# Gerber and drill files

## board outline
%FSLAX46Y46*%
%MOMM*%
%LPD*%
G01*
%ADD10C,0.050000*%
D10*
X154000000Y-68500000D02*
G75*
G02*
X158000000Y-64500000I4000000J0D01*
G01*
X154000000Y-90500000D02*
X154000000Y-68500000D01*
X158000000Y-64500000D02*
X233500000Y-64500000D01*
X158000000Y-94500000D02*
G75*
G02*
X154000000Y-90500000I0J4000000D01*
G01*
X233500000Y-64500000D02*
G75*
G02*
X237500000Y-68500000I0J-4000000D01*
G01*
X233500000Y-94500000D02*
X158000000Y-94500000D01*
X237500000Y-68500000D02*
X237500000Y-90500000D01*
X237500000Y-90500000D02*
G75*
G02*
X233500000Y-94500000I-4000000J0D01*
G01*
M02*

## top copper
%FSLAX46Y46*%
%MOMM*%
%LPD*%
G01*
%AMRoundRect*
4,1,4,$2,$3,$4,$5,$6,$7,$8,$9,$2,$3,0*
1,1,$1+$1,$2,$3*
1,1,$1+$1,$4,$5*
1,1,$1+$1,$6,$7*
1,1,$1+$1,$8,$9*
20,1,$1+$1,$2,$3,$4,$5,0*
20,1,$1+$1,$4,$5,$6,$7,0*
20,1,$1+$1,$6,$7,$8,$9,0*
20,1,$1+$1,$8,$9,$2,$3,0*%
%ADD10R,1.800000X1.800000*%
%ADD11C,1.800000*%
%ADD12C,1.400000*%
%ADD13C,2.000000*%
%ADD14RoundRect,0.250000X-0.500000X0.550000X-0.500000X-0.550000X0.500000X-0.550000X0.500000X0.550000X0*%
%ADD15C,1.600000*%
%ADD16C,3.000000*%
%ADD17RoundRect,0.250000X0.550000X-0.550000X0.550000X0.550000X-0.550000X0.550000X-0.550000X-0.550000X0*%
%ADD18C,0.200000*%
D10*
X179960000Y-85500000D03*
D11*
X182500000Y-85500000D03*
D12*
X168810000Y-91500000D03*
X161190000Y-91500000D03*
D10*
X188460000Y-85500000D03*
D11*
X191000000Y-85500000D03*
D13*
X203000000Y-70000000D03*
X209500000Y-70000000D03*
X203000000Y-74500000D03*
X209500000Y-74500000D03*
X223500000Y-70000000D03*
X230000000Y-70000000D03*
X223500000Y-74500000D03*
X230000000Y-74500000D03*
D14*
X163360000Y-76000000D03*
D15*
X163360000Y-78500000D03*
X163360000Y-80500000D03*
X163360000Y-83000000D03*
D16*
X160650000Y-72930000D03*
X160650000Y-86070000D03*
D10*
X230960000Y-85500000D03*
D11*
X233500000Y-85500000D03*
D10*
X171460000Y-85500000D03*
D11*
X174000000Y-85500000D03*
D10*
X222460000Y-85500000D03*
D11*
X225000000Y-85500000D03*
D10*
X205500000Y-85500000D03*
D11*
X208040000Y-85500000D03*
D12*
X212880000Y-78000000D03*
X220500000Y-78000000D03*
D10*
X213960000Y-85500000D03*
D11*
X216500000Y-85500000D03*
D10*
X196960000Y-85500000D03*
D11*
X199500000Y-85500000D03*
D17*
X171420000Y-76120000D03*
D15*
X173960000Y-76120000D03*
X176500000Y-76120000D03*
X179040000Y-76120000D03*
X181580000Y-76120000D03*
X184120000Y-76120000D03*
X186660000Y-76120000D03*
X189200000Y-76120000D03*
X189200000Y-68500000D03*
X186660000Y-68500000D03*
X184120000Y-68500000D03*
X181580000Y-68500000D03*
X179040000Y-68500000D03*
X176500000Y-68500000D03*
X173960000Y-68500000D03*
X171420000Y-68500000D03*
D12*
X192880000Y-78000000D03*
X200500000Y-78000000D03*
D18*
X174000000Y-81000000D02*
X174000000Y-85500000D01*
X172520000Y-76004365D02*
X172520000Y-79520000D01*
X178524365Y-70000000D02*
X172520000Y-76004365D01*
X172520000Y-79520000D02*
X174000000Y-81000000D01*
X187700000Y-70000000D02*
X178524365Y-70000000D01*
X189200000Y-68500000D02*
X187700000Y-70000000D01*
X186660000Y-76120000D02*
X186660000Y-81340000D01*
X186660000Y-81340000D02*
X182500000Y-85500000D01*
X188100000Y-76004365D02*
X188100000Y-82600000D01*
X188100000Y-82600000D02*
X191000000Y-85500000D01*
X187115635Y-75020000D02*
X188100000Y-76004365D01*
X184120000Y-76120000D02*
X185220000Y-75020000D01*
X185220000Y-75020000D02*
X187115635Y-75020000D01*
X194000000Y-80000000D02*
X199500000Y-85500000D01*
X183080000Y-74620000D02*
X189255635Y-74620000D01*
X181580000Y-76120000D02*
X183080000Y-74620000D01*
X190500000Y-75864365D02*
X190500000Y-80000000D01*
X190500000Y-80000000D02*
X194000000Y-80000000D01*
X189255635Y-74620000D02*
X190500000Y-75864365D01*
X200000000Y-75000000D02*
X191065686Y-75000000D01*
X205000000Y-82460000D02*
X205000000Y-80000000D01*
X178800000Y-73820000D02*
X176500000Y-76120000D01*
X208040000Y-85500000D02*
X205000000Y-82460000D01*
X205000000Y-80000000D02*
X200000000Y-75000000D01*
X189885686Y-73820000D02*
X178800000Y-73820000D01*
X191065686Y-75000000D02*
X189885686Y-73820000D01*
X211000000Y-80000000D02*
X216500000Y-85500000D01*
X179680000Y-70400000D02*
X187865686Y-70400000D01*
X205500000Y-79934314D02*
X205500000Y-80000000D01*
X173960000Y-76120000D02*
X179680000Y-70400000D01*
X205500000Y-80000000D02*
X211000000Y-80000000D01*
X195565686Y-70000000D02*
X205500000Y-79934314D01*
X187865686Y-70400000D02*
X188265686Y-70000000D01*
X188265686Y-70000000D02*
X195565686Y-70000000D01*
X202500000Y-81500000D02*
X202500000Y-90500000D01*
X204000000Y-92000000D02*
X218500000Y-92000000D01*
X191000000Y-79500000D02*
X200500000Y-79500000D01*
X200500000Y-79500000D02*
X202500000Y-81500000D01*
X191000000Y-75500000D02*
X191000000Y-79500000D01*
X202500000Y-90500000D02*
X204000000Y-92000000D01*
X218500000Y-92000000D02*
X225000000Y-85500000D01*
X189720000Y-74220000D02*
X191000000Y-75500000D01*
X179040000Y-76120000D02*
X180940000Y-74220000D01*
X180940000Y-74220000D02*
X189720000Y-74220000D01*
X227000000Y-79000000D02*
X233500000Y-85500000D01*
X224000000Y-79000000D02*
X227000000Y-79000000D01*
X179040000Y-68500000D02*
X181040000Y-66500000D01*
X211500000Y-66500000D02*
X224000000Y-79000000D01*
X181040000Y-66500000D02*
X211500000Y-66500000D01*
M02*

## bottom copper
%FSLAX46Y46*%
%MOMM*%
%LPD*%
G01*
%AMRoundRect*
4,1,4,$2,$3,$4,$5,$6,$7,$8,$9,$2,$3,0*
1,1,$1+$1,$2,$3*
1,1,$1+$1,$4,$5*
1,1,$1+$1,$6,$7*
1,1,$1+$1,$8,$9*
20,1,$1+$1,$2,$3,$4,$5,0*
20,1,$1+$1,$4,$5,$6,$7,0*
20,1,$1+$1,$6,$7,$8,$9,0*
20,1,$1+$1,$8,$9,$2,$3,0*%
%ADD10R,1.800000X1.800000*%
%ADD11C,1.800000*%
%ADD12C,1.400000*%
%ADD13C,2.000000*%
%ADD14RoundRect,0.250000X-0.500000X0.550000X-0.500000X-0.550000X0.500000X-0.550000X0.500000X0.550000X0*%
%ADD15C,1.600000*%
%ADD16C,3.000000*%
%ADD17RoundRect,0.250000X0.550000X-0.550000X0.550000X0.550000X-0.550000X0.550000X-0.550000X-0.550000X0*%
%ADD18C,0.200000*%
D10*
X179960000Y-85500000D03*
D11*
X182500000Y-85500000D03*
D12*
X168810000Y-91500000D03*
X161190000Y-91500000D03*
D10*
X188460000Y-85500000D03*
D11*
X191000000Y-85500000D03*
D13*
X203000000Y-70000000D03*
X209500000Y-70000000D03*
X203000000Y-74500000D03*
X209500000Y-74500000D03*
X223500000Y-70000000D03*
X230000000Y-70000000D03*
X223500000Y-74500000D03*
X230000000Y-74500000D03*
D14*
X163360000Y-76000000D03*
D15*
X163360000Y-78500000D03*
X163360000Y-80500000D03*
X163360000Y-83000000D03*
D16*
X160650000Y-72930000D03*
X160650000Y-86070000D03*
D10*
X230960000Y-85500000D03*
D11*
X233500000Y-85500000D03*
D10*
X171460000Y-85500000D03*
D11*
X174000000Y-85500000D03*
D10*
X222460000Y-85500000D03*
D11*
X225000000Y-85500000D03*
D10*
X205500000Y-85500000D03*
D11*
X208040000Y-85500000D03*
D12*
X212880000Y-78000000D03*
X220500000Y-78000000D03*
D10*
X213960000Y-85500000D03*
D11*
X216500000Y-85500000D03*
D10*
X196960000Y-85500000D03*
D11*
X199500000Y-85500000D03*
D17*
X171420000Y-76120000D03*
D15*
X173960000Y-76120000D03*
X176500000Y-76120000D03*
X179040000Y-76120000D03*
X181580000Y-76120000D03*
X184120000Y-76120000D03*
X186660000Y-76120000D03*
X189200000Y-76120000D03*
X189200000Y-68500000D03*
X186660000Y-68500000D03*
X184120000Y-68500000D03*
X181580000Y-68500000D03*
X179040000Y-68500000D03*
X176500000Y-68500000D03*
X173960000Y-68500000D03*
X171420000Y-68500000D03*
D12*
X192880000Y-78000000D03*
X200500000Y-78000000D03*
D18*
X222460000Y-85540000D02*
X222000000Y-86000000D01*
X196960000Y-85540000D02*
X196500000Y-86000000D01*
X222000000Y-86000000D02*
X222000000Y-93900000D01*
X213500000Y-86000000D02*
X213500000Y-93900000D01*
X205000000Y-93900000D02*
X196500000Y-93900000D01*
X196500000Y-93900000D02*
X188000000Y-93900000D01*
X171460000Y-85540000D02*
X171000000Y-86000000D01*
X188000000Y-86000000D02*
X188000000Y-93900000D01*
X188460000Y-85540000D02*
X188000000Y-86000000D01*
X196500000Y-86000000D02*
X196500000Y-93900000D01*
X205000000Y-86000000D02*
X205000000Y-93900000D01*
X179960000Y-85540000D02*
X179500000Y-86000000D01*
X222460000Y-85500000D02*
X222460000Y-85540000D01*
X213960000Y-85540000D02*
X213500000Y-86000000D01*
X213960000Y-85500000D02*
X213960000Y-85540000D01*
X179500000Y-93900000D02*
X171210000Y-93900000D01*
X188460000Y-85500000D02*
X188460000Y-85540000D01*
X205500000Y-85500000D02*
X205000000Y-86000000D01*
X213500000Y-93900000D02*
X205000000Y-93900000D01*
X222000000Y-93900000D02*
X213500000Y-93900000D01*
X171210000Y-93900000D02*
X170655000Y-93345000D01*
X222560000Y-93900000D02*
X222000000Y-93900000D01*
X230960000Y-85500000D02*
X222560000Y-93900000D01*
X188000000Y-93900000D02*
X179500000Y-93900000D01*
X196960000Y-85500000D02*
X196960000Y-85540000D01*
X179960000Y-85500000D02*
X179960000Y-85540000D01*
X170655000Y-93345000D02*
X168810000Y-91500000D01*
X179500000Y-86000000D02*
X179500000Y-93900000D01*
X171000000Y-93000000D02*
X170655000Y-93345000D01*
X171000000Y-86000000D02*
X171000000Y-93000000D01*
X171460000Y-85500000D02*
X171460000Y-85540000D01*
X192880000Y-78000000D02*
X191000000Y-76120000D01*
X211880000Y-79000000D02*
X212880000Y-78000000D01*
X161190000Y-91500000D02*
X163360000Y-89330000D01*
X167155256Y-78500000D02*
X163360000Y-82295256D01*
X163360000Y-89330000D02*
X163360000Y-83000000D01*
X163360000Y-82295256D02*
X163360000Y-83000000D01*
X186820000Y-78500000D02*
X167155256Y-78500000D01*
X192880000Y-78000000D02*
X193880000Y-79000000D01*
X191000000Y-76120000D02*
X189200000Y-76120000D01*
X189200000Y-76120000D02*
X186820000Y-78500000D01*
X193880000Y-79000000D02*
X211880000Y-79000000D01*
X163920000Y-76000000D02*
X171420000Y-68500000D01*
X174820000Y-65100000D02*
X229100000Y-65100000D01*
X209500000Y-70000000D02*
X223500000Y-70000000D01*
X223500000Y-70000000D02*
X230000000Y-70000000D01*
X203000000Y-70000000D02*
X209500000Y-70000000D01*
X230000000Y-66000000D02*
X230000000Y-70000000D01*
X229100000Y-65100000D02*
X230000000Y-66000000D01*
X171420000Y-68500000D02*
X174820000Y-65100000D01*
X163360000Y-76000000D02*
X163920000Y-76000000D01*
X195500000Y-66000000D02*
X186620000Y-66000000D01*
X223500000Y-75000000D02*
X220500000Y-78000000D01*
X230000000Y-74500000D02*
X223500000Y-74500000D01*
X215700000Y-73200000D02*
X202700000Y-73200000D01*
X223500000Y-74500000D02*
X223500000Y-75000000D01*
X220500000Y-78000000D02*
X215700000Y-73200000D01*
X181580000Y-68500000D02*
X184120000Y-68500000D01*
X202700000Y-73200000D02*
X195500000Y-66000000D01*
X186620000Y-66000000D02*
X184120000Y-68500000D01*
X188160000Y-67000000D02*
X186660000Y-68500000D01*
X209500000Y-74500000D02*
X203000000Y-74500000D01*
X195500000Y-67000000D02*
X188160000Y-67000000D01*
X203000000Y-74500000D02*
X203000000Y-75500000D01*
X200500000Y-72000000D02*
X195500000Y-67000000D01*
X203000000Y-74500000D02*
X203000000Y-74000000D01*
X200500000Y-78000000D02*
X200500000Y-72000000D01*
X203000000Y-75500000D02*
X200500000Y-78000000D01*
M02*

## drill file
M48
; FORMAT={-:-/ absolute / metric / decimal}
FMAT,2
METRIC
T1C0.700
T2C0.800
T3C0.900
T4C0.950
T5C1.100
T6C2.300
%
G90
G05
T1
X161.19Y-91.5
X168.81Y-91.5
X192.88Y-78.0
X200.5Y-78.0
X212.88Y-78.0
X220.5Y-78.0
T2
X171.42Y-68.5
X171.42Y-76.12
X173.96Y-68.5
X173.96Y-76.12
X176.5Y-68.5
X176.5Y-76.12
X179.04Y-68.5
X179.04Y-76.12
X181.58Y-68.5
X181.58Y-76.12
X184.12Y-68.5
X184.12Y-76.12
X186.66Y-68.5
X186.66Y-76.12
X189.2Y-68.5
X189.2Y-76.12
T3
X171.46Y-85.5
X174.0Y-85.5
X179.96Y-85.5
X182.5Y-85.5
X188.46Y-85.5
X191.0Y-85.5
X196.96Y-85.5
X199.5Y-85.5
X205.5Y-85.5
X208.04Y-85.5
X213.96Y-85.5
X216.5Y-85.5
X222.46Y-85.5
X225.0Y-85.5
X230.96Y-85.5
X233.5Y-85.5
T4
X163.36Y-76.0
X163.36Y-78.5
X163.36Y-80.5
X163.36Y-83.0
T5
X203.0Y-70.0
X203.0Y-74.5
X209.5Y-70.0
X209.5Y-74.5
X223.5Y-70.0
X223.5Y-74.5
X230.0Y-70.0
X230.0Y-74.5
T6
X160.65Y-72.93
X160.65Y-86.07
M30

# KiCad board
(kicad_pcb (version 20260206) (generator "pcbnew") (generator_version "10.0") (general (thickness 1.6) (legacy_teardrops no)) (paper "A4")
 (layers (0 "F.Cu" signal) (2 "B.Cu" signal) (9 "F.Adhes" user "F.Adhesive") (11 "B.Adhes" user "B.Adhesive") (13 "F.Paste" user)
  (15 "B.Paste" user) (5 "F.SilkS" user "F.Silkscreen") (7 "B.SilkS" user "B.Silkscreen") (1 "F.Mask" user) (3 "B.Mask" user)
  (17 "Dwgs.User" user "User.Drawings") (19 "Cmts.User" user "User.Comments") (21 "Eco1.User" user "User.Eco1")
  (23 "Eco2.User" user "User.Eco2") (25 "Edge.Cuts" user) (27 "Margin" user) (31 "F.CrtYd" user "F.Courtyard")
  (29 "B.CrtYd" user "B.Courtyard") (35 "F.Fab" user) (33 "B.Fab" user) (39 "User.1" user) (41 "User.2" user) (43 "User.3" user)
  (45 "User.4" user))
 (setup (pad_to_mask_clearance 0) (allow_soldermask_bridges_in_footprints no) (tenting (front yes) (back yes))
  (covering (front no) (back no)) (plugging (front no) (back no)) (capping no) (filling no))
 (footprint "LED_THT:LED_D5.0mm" (layer "F.Cu") (at 179.96 85.5)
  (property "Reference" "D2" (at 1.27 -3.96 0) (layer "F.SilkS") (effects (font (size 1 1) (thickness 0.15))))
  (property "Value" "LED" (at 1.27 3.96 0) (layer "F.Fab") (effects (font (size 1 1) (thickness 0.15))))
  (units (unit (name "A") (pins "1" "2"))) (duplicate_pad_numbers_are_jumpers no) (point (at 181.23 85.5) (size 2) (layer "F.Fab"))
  (pad "1" thru_hole rect (at 0 0) (size 1.8 1.8) (drill 0.9) (layers "*.Cu" "*.Mask") (remove_unused_layers no) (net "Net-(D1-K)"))
  (pad "2" thru_hole circle (at 2.54 0) (size 1.8 1.8) (drill 0.9) (layers "*.Cu" "*.Mask") (remove_unused_layers no) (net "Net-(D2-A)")))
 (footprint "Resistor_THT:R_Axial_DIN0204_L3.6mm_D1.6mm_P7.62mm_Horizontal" (layer "F.Cu") (at 168.81 91.5 180)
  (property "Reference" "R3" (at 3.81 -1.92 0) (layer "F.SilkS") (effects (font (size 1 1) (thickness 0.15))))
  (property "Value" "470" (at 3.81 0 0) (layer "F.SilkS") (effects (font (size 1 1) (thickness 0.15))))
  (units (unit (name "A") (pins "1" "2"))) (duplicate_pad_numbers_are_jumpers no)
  (pad "1" thru_hole circle (at 0 0 180) (size 1.4 1.4) (drill 0.7) (layers "*.Cu" "*.Mask") (remove_unused_layers no) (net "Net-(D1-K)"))
  (pad "2" thru_hole circle (at 7.62 0 180) (size 1.4 1.4) (drill 0.7) (layers "*.Cu" "*.Mask") (remove_unused_layers no) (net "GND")))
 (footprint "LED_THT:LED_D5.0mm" (layer "F.Cu") (at 188.46 85.5)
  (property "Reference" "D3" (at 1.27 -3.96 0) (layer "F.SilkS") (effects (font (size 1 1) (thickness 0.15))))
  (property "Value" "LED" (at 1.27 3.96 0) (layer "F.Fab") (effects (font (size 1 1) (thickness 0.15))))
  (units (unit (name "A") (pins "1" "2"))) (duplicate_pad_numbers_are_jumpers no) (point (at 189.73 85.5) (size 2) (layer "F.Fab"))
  (pad "1" thru_hole rect (at 0 0) (size 1.8 1.8) (drill 0.9) (layers "*.Cu" "*.Mask") (remove_unused_layers no) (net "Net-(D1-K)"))
  (pad "2" thru_hole circle (at 2.54 0) (size 1.8 1.8) (drill 0.9) (layers "*.Cu" "*.Mask") (remove_unused_layers no) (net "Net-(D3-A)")))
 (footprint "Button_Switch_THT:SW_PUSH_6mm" (layer "F.Cu") (at 203 70)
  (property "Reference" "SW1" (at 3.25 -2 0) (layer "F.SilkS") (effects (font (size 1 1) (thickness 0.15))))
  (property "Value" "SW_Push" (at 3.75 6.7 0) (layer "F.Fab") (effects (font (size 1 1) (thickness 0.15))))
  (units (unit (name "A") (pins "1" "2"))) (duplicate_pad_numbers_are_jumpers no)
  (pad "1" thru_hole circle (at 0 0 90) (size 2 2) (drill 1.1) (layers "*.Cu" "*.Mask") (remove_unused_layers no) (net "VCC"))
  (pad "1" thru_hole circle (at 6.5 0 90) (size 2 2) (drill 1.1) (layers "*.Cu" "*.Mask") (remove_unused_layers no) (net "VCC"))
  (pad "2" thru_hole circle (at 0 4.5 90) (size 2 2) (drill 1.1) (layers "*.Cu" "*.Mask") (remove_unused_layers no) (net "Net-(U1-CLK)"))
  (pad "2" thru_hole circle (at 6.5 4.5 90) (size 2 2) (drill 1.1) (layers "*.Cu" "*.Mask") (remove_unused_layers no) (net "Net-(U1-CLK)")))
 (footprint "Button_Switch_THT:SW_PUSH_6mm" (layer "F.Cu") (at 223.5 70)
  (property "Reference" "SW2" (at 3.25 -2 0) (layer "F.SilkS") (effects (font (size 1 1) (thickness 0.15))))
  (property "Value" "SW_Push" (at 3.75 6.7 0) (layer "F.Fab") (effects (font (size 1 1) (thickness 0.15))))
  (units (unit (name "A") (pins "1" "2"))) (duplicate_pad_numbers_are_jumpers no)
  (pad "1" thru_hole circle (at 0 0 90) (size 2 2) (drill 1.1) (layers "*.Cu" "*.Mask") (remove_unused_layers no) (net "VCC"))
  (pad "1" thru_hole circle (at 6.5 0 90) (size 2 2) (drill 1.1) (layers "*.Cu" "*.Mask") (remove_unused_layers no) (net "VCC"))
  (pad "2" thru_hole circle (at 0 4.5 90) (size 2 2) (drill 1.1) (layers "*.Cu" "*.Mask") (remove_unused_layers no) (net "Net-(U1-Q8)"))
  (pad "2" thru_hole circle (at 6.5 4.5 90) (size 2 2) (drill 1.1) (layers "*.Cu" "*.Mask") (remove_unused_layers no) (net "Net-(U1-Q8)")))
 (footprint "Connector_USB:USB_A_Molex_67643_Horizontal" (layer "F.Cu") (at 163.36 76 -90)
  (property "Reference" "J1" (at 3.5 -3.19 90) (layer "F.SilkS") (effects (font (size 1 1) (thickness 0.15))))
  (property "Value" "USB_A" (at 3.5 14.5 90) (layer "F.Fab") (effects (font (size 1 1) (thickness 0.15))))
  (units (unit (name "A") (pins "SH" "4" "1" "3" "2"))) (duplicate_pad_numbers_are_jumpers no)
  (pad "1" thru_hole roundrect (at 0 0 270) (size 1.6 1.5) (drill 0.95) (layers "*.Cu" "*.Mask") (remove_unused_layers no)
   (roundrect_rratio 0.1666666667) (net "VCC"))
  (pad "2" thru_hole circle (at 2.5 0 270) (size 1.6 1.6) (drill 0.95) (layers "*.Cu" "*.Mask") (remove_unused_layers no)
   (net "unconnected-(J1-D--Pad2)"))
  (pad "3" thru_hole circle (at 4.5 0 270) (size 1.6 1.6) (drill 0.95) (layers "*.Cu" "*.Mask") (remove_unused_layers no)
   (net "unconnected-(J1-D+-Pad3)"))
  (pad "4" thru_hole circle (at 7 0 270) (size 1.6 1.6) (drill 0.95) (layers "*.Cu" "*.Mask") (remove_unused_layers no) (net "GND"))
  (pad "SH" thru_hole circle (at -3.07 2.71 270) (size 3 3) (drill 2.3) (layers "*.Cu" "*.Mask") (remove_unused_layers no)
   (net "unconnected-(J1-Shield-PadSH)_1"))
  (pad "SH" thru_hole circle (at 10.07 2.71 270) (size 3 3) (drill 2.3) (layers "*.Cu" "*.Mask") (remove_unused_layers no)
   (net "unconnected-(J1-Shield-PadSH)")))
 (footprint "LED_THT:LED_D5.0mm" (layer "F.Cu") (at 230.96 85.5)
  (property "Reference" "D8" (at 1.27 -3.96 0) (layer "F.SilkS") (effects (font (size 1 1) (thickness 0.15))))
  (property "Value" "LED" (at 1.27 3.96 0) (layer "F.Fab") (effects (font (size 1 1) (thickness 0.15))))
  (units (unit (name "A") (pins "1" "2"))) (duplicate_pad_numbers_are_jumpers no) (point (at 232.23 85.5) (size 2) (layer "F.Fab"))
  (pad "1" thru_hole rect (at 0 0) (size 1.8 1.8) (drill 0.9) (layers "*.Cu" "*.Mask") (remove_unused_layers no) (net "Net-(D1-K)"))
  (pad "2" thru_hole circle (at 2.54 0) (size 1.8 1.8) (drill 0.9) (layers "*.Cu" "*.Mask") (remove_unused_layers no) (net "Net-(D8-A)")))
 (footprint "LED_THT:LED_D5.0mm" (layer "F.Cu") (at 171.46 85.5)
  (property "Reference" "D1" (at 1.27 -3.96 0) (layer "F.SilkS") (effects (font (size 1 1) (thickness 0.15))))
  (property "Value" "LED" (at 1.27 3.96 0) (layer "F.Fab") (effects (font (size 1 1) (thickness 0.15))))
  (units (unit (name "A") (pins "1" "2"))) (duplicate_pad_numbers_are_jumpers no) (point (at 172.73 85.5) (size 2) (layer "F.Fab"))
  (pad "1" thru_hole rect (at 0 0) (size 1.8 1.8) (drill 0.9) (layers "*.Cu" "*.Mask") (remove_unused_layers no) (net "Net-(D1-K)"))
  (pad "2" thru_hole circle (at 2.54 0) (size 1.8 1.8) (drill 0.9) (layers "*.Cu" "*.Mask") (remove_unused_layers no) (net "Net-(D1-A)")))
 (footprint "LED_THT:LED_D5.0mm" (layer "F.Cu") (at 222.46 85.5)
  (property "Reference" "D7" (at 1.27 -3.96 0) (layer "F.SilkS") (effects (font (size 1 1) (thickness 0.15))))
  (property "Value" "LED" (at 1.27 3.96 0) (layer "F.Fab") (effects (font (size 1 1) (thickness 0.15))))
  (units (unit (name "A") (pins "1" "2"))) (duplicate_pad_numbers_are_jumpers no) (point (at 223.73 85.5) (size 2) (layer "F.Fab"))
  (pad "1" thru_hole rect (at 0 0) (size 1.8 1.8) (drill 0.9) (layers "*.Cu" "*.Mask") (remove_unused_layers no) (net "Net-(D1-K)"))
  (pad "2" thru_hole circle (at 2.54 0) (size 1.8 1.8) (drill 0.9) (layers "*.Cu" "*.Mask") (remove_unused_layers no) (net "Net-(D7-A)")))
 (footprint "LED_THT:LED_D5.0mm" (layer "F.Cu") (at 205.5 85.5)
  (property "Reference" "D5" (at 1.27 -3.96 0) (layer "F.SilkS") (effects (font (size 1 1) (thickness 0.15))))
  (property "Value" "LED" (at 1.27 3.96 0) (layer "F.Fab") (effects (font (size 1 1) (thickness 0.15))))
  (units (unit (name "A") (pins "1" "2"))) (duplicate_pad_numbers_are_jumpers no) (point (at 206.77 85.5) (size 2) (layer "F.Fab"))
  (pad "1" thru_hole rect (at 0 0) (size 1.8 1.8) (drill 0.9) (layers "*.Cu" "*.Mask") (remove_unused_layers no) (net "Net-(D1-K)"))
  (pad "2" thru_hole circle (at 2.54 0) (size 1.8 1.8) (drill 0.9) (layers "*.Cu" "*.Mask") (remove_unused_layers no) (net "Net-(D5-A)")))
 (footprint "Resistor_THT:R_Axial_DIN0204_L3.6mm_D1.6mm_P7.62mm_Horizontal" (layer "F.Cu") (at 212.88 78)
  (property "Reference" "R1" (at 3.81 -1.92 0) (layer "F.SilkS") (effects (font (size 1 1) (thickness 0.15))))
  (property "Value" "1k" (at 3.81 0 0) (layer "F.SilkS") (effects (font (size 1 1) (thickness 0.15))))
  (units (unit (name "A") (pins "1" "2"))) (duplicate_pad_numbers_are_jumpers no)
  (pad "1" thru_hole circle (at 0 0) (size 1.4 1.4) (drill 0.7) (layers "*.Cu" "*.Mask") (remove_unused_layers no) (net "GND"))
  (pad "2" thru_hole circle (at 7.62 0) (size 1.4 1.4) (drill 0.7) (layers "*.Cu" "*.Mask") (remove_unused_layers no) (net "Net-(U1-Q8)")))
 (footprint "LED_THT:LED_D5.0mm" (layer "F.Cu") (at 213.96 85.5)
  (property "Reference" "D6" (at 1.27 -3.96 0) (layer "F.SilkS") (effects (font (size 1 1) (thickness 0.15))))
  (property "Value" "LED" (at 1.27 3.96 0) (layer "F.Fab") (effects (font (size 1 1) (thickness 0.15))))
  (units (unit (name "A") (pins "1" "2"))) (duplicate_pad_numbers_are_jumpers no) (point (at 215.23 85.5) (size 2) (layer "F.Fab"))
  (pad "1" thru_hole rect (at 0 0) (size 1.8 1.8) (drill 0.9) (layers "*.Cu" "*.Mask") (remove_unused_layers no) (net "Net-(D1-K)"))
  (pad "2" thru_hole circle (at 2.54 0) (size 1.8 1.8) (drill 0.9) (layers "*.Cu" "*.Mask") (remove_unused_layers no) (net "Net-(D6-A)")))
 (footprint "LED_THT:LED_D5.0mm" (layer "F.Cu") (at 196.96 85.5)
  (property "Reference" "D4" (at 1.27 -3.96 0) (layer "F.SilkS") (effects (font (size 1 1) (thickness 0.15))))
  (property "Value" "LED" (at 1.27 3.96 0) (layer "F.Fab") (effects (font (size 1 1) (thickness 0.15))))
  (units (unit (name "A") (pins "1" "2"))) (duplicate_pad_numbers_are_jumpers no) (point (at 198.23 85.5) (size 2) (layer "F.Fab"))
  (pad "1" thru_hole rect (at 0 0) (size 1.8 1.8) (drill 0.9) (layers "*.Cu" "*.Mask") (remove_unused_layers no) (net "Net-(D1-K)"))
  (pad "2" thru_hole circle (at 2.54 0) (size 1.8 1.8) (drill 0.9) (layers "*.Cu" "*.Mask") (remove_unused_layers no) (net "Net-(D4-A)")))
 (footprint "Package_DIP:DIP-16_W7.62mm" (layer "F.Cu") (at 171.42 76.12 90)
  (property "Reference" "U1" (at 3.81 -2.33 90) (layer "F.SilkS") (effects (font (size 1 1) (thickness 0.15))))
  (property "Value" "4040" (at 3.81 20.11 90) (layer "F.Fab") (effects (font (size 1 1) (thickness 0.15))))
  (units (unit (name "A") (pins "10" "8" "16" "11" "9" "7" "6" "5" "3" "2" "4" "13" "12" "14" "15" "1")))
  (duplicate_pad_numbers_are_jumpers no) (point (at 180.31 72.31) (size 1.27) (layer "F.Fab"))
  (pad "1" thru_hole roundrect (at 0 0 90) (size 1.6 1.6) (drill 0.8) (layers "*.Cu" "*.Mask") (remove_unused_layers no)
   (roundrect_rratio 0.15625) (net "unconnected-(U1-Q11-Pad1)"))
  (pad "2" thru_hole circle (at 0 2.54 90) (size 1.6 1.6) (drill 0.8) (layers "*.Cu" "*.Mask") (remove_unused_layers no) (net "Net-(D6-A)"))
  (pad "3" thru_hole circle (at 0 5.08 90) (size 1.6 1.6) (drill 0.8) (layers "*.Cu" "*.Mask") (remove_unused_layers no) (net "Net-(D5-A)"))
  (pad "4" thru_hole circle (at 0 7.62 90) (size 1.6 1.6) (drill 0.8) (layers "*.Cu" "*.Mask") (remove_unused_layers no) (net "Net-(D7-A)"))
  (pad "5" thru_hole circle (at 0 10.16 90) (size 1.6 1.6) (drill 0.8) (layers "*.Cu" "*.Mask") (remove_unused_layers no) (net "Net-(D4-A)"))
  (pad "6" thru_hole circle (at 0 12.7 90) (size 1.6 1.6) (drill 0.8) (layers "*.Cu" "*.Mask") (remove_unused_layers no) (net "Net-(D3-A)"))
  (pad "7" thru_hole circle (at 0 15.24 90) (size 1.6 1.6) (drill 0.8) (layers "*.Cu" "*.Mask") (remove_unused_layers no) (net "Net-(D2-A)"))
  (pad "8" thru_hole circle (at 0 17.78 90) (size 1.6 1.6) (drill 0.8) (layers "*.Cu" "*.Mask") (remove_unused_layers no) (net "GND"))
  (pad "9" thru_hole circle (at 7.62 17.78 90) (size 1.6 1.6) (drill 0.8) (layers "*.Cu" "*.Mask") (remove_unused_layers no)
   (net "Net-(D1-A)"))
  (pad "10" thru_hole circle (at 7.62 15.24 90) (size 1.6 1.6) (drill 0.8) (layers "*.Cu" "*.Mask") (remove_unused_layers no)
   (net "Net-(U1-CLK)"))
  (pad "11" thru_hole circle (at 7.62 12.7 90) (size 1.6 1.6) (drill 0.8) (layers "*.Cu" "*.Mask") (remove_unused_layers no)
   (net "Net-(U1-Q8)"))
  (pad "12" thru_hole circle (at 7.62 10.16 90) (size 1.6 1.6) (drill 0.8) (layers "*.Cu" "*.Mask") (remove_unused_layers no)
   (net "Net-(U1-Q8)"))
  (pad "13" thru_hole circle (at 7.62 7.62 90) (size 1.6 1.6) (drill 0.8) (layers "*.Cu" "*.Mask") (remove_unused_layers no)
   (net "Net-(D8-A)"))
  (pad "14" thru_hole circle (at 7.62 5.08 90) (size 1.6 1.6) (drill 0.8) (layers "*.Cu" "*.Mask") (remove_unused_layers no)
   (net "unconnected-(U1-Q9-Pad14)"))
  (pad "15" thru_hole circle (at 7.62 2.54 90) (size 1.6 1.6) (drill 0.8) (layers "*.Cu" "*.Mask") (remove_unused_layers no)
   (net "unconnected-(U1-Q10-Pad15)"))
  (pad "16" thru_hole circle (at 7.62 0 90) (size 1.6 1.6) (drill 0.8) (layers "*.Cu" "*.Mask") (remove_unused_layers no) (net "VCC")))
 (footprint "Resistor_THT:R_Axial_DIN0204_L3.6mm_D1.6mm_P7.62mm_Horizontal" (layer "F.Cu") (at 192.88 78)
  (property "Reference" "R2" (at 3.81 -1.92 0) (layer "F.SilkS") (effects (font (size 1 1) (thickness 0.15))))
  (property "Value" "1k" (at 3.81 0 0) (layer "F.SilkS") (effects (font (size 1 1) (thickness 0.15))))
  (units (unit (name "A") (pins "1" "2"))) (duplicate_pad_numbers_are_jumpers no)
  (pad "1" thru_hole circle (at 0 0) (size 1.4 1.4) (drill 0.7) (layers "*.Cu" "*.Mask") (remove_unused_layers no) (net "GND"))
  (pad "2" thru_hole circle (at 7.62 0) (size 1.4 1.4) (drill 0.7) (layers "*.Cu" "*.Mask") (remove_unused_layers no) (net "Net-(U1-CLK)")))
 (gr_arc (start 154 68.5) (mid 155.171573 65.671573) (end 158 64.5) (stroke (width 0.05) (type default)) (layer "Edge.Cuts"))
 (gr_line (start 154 90.5) (end 154 68.5) (stroke (width 0.05) (type default)) (layer "Edge.Cuts"))
 (gr_line (start 158 64.5) (end 233.5 64.5) (stroke (width 0.05) (type default)) (layer "Edge.Cuts"))
 (gr_arc (start 158 94.5) (mid 155.171573 93.328427) (end 154 90.5) (stroke (width 0.05) (type default)) (layer "Edge.Cuts"))
 (gr_arc (start 233.5 64.5) (mid 236.328427 65.671573) (end 237.5 68.5) (stroke (width 0.05) (type default)) (layer "Edge.Cuts"))
 (gr_line (start 233.5 94.5) (end 158 94.5) (stroke (width 0.05) (type default)) (layer "Edge.Cuts"))
 (gr_line (start 237.5 68.5) (end 237.5 90.5) (stroke (width 0.05) (type default)) (layer "Edge.Cuts"))
 (gr_arc (start 237.5 90.5) (mid 236.328427 93.328427) (end 233.5 94.5) (stroke (width 0.05) (type default)) (layer "Edge.Cuts"))
 (segment (start 222.46 85.54) (end 222 86) (width 0.2) (layer "B.Cu") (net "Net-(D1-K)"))
 (segment (start 196.96 85.54) (end 196.5 86) (width 0.2) (layer "B.Cu") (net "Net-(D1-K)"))
 (segment (start 222 86) (end 222 93.9) (width 0.2) (layer "B.Cu") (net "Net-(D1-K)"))
 (segment (start 213.5 86) (end 213.5 93.9) (width 0.2) (layer "B.Cu") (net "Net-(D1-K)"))
 (segment (start 205 93.9) (end 196.5 93.9) (width 0.2) (layer "B.Cu") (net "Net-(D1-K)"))
 (segment (start 196.5 93.9) (end 188 93.9) (width 0.2) (layer "B.Cu") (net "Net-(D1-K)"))
 (segment (start 171.46 85.54) (end 171 86) (width 0.2) (layer "B.Cu") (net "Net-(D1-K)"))
 (segment (start 188 86) (end 188 93.9) (width 0.2) (layer "B.Cu") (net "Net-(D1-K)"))
 (segment (start 188.46 85.54) (end 188 86) (width 0.2) (layer "B.Cu") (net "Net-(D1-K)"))
 (segment (start 196.5 86) (end 196.5 93.9) (width 0.2) (layer "B.Cu") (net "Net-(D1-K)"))
 (segment (start 205 86) (end 205 93.9) (width 0.2) (layer "B.Cu") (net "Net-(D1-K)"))
 (segment (start 179.96 85.54) (end 179.5 86) (width 0.2) (layer "B.Cu") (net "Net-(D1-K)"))
 (segment (start 222.46 85.5) (end 222.46 85.54) (width 0.2) (layer "B.Cu") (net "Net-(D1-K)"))
 (segment (start 213.96 85.54) (end 213.5 86) (width 0.2) (layer "B.Cu") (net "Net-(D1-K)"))
 (segment (start 213.96 85.5) (end 213.96 85.54) (width 0.2) (layer "B.Cu") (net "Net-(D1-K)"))
 (segment (start 179.5 93.9) (end 171.21 93.9) (width 0.2) (layer "B.Cu") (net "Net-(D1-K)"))
 (segment (start 188.46 85.5) (end 188.46 85.54) (width 0.2) (layer "B.Cu") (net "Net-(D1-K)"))
 (segment (start 205.5 85.5) (end 205 86) (width 0.2) (layer "B.Cu") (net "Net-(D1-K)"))
 (segment (start 213.5 93.9) (end 205 93.9) (width 0.2) (layer "B.Cu") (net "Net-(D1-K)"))
 (segment (start 222 93.9) (end 213.5 93.9) (width 0.2) (layer "B.Cu") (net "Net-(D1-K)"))
 (segment (start 171.21 93.9) (end 170.655 93.345) (width 0.2) (layer "B.Cu") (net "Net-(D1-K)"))
 (segment (start 222.56 93.9) (end 222 93.9) (width 0.2) (layer "B.Cu") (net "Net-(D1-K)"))
 (segment (start 230.96 85.5) (end 222.56 93.9) (width 0.2) (layer "B.Cu") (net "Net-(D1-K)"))
 (segment (start 188 93.9) (end 179.5 93.9) (width 0.2) (layer "B.Cu") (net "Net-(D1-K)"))
 (segment (start 196.96 85.5) (end 196.96 85.54) (width 0.2) (layer "B.Cu") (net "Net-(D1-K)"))
 (segment (start 179.96 85.5) (end 179.96 85.54) (width 0.2) (layer "B.Cu") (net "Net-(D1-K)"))
 (segment (start 170.655 93.345) (end 168.81 91.5) (width 0.2) (layer "B.Cu") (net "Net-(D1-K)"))
 (segment (start 179.5 86) (end 179.5 93.9) (width 0.2) (layer "B.Cu") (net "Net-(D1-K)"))
 (segment (start 171 93) (end 170.655 93.345) (width 0.2) (layer "B.Cu") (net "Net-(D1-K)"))
 (segment (start 171 86) (end 171 93) (width 0.2) (layer "B.Cu") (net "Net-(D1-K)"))
 (segment (start 171.46 85.5) (end 171.46 85.54) (width 0.2) (layer "B.Cu") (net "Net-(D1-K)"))
 (segment (start 174 81) (end 174 85.5) (width 0.2) (layer "F.Cu") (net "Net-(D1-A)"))
 (segment (start 172.52 76.004365) (end 172.52 79.52) (width 0.2) (layer "F.Cu") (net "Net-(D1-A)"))
 (segment (start 178.524365 70) (end 172.52 76.004365) (width 0.2) (layer "F.Cu") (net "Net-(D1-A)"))
 (segment (start 172.52 79.52) (end 174 81) (width 0.2) (layer "F.Cu") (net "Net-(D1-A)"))
 (segment (start 187.7 70) (end 178.524365 70) (width 0.2) (layer "F.Cu") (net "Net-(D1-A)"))
 (segment (start 189.2 68.5) (end 187.7 70) (width 0.2) (layer "F.Cu") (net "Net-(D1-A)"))
 (segment (start 186.66 76.12) (end 186.66 81.34) (width 0.2) (layer "F.Cu") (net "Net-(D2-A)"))
 (segment (start 186.66 81.34) (end 182.5 85.5) (width 0.2) (layer "F.Cu") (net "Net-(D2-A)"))
 (segment (start 188.1 76.004365) (end 188.1 82.6) (width 0.2) (layer "F.Cu") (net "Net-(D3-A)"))
 (segment (start 188.1 82.6) (end 191 85.5) (width 0.2) (layer "F.Cu") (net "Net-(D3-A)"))
 (segment (start 187.115635 75.02) (end 188.1 76.004365) (width 0.2) (layer "F.Cu") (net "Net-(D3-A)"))
 (segment (start 184.12 76.12) (end 185.22 75.02) (width 0.2) (layer "F.Cu") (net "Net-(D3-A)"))
 (segment (start 185.22 75.02) (end 187.115635 75.02) (width 0.2) (layer "F.Cu") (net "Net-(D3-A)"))
 (segment (start 194 80) (end 199.5 85.5) (width 0.2) (layer "F.Cu") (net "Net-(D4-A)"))
 (segment (start 183.08 74.62) (end 189.255635 74.62) (width 0.2) (layer "F.Cu") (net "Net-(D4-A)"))
 (segment (start 181.58 76.12) (end 183.08 74.62) (width 0.2) (layer "F.Cu") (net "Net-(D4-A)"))
 (segment (start 190.5 75.864365) (end 190.5 80) (width 0.2) (layer "F.Cu") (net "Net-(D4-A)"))
 (segment (start 190.5 80) (end 194 80) (width 0.2) (layer "F.Cu") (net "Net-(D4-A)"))
 (segment (start 189.255635 74.62) (end 190.5 75.864365) (width 0.2) (layer "F.Cu") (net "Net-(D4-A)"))
 (segment (start 200 75) (end 191.065686 75) (width 0.2) (layer "F.Cu") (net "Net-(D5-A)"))
 (segment (start 205 82.46) (end 205 80) (width 0.2) (layer "F.Cu") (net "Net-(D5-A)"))
 (segment (start 178.8 73.82) (end 176.5 76.12) (width 0.2) (layer "F.Cu") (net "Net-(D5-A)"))
 (segment (start 208.04 85.5) (end 205 82.46) (width 0.2) (layer "F.Cu") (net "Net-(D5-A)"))
 (segment (start 205 80) (end 200 75) (width 0.2) (layer "F.Cu") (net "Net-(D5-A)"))
 (segment (start 189.885686 73.82) (end 178.8 73.82) (width 0.2) (layer "F.Cu") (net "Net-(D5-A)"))
 (segment (start 191.065686 75) (end 189.885686 73.82) (width 0.2) (layer "F.Cu") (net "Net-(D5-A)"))
 (segment (start 211 80) (end 216.5 85.5) (width 0.2) (layer "F.Cu") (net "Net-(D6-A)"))
 (segment (start 179.68 70.4) (end 187.865686 70.4) (width 0.2) (layer "F.Cu") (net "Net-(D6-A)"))
 (segment (start 205.5 79.934314) (end 205.5 80) (width 0.2) (layer "F.Cu") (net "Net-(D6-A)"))
 (segment (start 173.96 76.12) (end 179.68 70.4) (width 0.2) (layer "F.Cu") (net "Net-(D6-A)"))
 (segment (start 205.5 80) (end 211 80) (width 0.2) (layer "F.Cu") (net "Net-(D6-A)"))
 (segment (start 195.565686 70) (end 205.5 79.934314) (width 0.2) (layer "F.Cu") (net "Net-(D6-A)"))
 (segment (start 187.865686 70.4) (end 188.265686 70) (width 0.2) (layer "F.Cu") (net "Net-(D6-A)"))
 (segment (start 188.265686 70) (end 195.565686 70) (width 0.2) (layer "F.Cu") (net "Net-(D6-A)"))
 (segment (start 202.5 81.5) (end 202.5 90.5) (width 0.2) (layer "F.Cu") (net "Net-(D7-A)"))
 (segment (start 204 92) (end 218.5 92) (width 0.2) (layer "F.Cu") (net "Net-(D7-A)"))
 (segment (start 191 79.5) (end 200.5 79.5) (width 0.2) (layer "F.Cu") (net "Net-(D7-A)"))
 (segment (start 200.5 79.5) (end 202.5 81.5) (width 0.2) (layer "F.Cu") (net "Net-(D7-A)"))
 (segment (start 191 75.5) (end 191 79.5) (width 0.2) (layer "F.Cu") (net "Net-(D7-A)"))
 (segment (start 202.5 90.5) (end 204 92) (width 0.2) (layer "F.Cu") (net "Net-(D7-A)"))
 (segment (start 218.5 92) (end 225 85.5) (width 0.2) (layer "F.Cu") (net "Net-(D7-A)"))
 (segment (start 189.72 74.22) (end 191 75.5) (width 0.2) (layer "F.Cu") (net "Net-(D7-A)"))
 (segment (start 179.04 76.12) (end 180.94 74.22) (width 0.2) (layer "F.Cu") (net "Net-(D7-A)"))
 (segment (start 180.94 74.22) (end 189.72 74.22) (width 0.2) (layer "F.Cu") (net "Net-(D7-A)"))
 (segment (start 227 79) (end 233.5 85.5) (width 0.2) (layer "F.Cu") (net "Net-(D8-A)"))
 (segment (start 224 79) (end 227 79) (width 0.2) (layer "F.Cu") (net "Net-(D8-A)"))
 (segment (start 179.04 68.5) (end 181.04 66.5) (width 0.2) (layer "F.Cu") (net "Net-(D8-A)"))
 (segment (start 211.5 66.5) (end 224 79) (width 0.2) (layer "F.Cu") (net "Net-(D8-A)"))
 (segment (start 181.04 66.5) (end 211.5 66.5) (width 0.2) (layer "F.Cu") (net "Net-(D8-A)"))
 (segment (start 192.88 78) (end 191 76.12) (width 0.2) (layer "B.Cu") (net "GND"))
 (segment (start 211.88 79) (end 212.88 78) (width 0.2) (layer "B.Cu") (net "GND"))
 (segment (start 161.19 91.5) (end 163.36 89.33) (width 0.2) (layer "B.Cu") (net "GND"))
 (segment (start 167.155256 78.5) (end 163.36 82.295256) (width 0.2) (layer "B.Cu") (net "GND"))
 (segment (start 163.36 89.33) (end 163.36 83) (width 0.2) (layer "B.Cu") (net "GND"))
 (segment (start 163.36 82.295256) (end 163.36 83) (width 0.2) (layer "B.Cu") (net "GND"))
 (segment (start 186.82 78.5) (end 167.155256 78.5) (width 0.2) (layer "B.Cu") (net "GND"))
 (segment (start 192.88 78) (end 193.88 79) (width 0.2) (layer "B.Cu") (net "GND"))
 (segment (start 191 76.12) (end 189.2 76.12) (width 0.2) (layer "B.Cu") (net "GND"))
 (segment (start 189.2 76.12) (end 186.82 78.5) (width 0.2) (layer "B.Cu") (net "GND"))
 (segment (start 193.88 79) (end 211.88 79) (width 0.2) (layer "B.Cu") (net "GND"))
 (segment (start 163.92 76) (end 171.42 68.5) (width 0.2) (layer "B.Cu") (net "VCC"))
 (segment (start 174.82 65.1) (end 229.1 65.1) (width 0.2) (layer "B.Cu") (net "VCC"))
 (segment (start 209.5 70) (end 223.5 70) (width 0.2) (layer "B.Cu") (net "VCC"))
 (segment (start 223.5 70) (end 230 70) (width 0.2) (layer "B.Cu") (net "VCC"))
 (segment (start 203 70) (end 209.5 70) (width 0.2) (layer "B.Cu") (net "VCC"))
 (segment (start 230 66) (end 230 70) (width 0.2) (layer "B.Cu") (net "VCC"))
 (segment (start 229.1 65.1) (end 230 66) (width 0.2) (layer "B.Cu") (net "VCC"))
 (segment (start 171.42 68.5) (end 174.82 65.1) (width 0.2) (layer "B.Cu") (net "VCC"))
 (segment (start 163.36 76) (end 163.92 76) (width 0.2) (layer "B.Cu") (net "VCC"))
 (segment (start 195.5 66) (end 186.62 66) (width 0.2) (layer "B.Cu") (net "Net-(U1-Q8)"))
 (segment (start 223.5 75) (end 220.5 78) (width 0.2) (layer "B.Cu") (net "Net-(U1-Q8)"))
 (segment (start 230 74.5) (end 223.5 74.5) (width 0.2) (layer "B.Cu") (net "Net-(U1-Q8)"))
 (segment (start 215.7 73.2) (end 202.7 73.2) (width 0.2) (layer "B.Cu") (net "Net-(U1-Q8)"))
 (segment (start 223.5 74.5) (end 223.5 75) (width 0.2) (layer "B.Cu") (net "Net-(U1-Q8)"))
 (segment (start 220.5 78) (end 215.7 73.2) (width 0.2) (layer "B.Cu") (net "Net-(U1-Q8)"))
 (segment (start 181.58 68.5) (end 184.12 68.5) (width 0.2) (layer "B.Cu") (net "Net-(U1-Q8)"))
 (segment (start 202.7 73.2) (end 195.5 66) (width 0.2) (layer "B.Cu") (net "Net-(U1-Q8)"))
 (segment (start 186.62 66) (end 184.12 68.5) (width 0.2) (layer "B.Cu") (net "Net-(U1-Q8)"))
 (segment (start 188.16 67) (end 186.66 68.5) (width 0.2) (layer "B.Cu") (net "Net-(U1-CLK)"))
 (segment (start 209.5 74.5) (end 203 74.5) (width 0.2) (layer "B.Cu") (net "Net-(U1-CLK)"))
 (segment (start 195.5 67) (end 188.16 67) (width 0.2) (layer "B.Cu") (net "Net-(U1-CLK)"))
 (segment (start 203 74.5) (end 203 75.5) (width 0.2) (layer "B.Cu") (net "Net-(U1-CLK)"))
 (segment (start 200.5 72) (end 195.5 67) (width 0.2) (layer "B.Cu") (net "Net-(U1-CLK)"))
 (segment (start 203 74.5) (end 203 74) (width 0.2) (layer "B.Cu") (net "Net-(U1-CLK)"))
 (segment (start 200.5 78) (end 200.5 72) (width 0.2) (layer "B.Cu") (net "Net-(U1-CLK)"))
 (segment (start 203 75.5) (end 200.5 78) (width 0.2) (layer "B.Cu") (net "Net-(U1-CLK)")))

